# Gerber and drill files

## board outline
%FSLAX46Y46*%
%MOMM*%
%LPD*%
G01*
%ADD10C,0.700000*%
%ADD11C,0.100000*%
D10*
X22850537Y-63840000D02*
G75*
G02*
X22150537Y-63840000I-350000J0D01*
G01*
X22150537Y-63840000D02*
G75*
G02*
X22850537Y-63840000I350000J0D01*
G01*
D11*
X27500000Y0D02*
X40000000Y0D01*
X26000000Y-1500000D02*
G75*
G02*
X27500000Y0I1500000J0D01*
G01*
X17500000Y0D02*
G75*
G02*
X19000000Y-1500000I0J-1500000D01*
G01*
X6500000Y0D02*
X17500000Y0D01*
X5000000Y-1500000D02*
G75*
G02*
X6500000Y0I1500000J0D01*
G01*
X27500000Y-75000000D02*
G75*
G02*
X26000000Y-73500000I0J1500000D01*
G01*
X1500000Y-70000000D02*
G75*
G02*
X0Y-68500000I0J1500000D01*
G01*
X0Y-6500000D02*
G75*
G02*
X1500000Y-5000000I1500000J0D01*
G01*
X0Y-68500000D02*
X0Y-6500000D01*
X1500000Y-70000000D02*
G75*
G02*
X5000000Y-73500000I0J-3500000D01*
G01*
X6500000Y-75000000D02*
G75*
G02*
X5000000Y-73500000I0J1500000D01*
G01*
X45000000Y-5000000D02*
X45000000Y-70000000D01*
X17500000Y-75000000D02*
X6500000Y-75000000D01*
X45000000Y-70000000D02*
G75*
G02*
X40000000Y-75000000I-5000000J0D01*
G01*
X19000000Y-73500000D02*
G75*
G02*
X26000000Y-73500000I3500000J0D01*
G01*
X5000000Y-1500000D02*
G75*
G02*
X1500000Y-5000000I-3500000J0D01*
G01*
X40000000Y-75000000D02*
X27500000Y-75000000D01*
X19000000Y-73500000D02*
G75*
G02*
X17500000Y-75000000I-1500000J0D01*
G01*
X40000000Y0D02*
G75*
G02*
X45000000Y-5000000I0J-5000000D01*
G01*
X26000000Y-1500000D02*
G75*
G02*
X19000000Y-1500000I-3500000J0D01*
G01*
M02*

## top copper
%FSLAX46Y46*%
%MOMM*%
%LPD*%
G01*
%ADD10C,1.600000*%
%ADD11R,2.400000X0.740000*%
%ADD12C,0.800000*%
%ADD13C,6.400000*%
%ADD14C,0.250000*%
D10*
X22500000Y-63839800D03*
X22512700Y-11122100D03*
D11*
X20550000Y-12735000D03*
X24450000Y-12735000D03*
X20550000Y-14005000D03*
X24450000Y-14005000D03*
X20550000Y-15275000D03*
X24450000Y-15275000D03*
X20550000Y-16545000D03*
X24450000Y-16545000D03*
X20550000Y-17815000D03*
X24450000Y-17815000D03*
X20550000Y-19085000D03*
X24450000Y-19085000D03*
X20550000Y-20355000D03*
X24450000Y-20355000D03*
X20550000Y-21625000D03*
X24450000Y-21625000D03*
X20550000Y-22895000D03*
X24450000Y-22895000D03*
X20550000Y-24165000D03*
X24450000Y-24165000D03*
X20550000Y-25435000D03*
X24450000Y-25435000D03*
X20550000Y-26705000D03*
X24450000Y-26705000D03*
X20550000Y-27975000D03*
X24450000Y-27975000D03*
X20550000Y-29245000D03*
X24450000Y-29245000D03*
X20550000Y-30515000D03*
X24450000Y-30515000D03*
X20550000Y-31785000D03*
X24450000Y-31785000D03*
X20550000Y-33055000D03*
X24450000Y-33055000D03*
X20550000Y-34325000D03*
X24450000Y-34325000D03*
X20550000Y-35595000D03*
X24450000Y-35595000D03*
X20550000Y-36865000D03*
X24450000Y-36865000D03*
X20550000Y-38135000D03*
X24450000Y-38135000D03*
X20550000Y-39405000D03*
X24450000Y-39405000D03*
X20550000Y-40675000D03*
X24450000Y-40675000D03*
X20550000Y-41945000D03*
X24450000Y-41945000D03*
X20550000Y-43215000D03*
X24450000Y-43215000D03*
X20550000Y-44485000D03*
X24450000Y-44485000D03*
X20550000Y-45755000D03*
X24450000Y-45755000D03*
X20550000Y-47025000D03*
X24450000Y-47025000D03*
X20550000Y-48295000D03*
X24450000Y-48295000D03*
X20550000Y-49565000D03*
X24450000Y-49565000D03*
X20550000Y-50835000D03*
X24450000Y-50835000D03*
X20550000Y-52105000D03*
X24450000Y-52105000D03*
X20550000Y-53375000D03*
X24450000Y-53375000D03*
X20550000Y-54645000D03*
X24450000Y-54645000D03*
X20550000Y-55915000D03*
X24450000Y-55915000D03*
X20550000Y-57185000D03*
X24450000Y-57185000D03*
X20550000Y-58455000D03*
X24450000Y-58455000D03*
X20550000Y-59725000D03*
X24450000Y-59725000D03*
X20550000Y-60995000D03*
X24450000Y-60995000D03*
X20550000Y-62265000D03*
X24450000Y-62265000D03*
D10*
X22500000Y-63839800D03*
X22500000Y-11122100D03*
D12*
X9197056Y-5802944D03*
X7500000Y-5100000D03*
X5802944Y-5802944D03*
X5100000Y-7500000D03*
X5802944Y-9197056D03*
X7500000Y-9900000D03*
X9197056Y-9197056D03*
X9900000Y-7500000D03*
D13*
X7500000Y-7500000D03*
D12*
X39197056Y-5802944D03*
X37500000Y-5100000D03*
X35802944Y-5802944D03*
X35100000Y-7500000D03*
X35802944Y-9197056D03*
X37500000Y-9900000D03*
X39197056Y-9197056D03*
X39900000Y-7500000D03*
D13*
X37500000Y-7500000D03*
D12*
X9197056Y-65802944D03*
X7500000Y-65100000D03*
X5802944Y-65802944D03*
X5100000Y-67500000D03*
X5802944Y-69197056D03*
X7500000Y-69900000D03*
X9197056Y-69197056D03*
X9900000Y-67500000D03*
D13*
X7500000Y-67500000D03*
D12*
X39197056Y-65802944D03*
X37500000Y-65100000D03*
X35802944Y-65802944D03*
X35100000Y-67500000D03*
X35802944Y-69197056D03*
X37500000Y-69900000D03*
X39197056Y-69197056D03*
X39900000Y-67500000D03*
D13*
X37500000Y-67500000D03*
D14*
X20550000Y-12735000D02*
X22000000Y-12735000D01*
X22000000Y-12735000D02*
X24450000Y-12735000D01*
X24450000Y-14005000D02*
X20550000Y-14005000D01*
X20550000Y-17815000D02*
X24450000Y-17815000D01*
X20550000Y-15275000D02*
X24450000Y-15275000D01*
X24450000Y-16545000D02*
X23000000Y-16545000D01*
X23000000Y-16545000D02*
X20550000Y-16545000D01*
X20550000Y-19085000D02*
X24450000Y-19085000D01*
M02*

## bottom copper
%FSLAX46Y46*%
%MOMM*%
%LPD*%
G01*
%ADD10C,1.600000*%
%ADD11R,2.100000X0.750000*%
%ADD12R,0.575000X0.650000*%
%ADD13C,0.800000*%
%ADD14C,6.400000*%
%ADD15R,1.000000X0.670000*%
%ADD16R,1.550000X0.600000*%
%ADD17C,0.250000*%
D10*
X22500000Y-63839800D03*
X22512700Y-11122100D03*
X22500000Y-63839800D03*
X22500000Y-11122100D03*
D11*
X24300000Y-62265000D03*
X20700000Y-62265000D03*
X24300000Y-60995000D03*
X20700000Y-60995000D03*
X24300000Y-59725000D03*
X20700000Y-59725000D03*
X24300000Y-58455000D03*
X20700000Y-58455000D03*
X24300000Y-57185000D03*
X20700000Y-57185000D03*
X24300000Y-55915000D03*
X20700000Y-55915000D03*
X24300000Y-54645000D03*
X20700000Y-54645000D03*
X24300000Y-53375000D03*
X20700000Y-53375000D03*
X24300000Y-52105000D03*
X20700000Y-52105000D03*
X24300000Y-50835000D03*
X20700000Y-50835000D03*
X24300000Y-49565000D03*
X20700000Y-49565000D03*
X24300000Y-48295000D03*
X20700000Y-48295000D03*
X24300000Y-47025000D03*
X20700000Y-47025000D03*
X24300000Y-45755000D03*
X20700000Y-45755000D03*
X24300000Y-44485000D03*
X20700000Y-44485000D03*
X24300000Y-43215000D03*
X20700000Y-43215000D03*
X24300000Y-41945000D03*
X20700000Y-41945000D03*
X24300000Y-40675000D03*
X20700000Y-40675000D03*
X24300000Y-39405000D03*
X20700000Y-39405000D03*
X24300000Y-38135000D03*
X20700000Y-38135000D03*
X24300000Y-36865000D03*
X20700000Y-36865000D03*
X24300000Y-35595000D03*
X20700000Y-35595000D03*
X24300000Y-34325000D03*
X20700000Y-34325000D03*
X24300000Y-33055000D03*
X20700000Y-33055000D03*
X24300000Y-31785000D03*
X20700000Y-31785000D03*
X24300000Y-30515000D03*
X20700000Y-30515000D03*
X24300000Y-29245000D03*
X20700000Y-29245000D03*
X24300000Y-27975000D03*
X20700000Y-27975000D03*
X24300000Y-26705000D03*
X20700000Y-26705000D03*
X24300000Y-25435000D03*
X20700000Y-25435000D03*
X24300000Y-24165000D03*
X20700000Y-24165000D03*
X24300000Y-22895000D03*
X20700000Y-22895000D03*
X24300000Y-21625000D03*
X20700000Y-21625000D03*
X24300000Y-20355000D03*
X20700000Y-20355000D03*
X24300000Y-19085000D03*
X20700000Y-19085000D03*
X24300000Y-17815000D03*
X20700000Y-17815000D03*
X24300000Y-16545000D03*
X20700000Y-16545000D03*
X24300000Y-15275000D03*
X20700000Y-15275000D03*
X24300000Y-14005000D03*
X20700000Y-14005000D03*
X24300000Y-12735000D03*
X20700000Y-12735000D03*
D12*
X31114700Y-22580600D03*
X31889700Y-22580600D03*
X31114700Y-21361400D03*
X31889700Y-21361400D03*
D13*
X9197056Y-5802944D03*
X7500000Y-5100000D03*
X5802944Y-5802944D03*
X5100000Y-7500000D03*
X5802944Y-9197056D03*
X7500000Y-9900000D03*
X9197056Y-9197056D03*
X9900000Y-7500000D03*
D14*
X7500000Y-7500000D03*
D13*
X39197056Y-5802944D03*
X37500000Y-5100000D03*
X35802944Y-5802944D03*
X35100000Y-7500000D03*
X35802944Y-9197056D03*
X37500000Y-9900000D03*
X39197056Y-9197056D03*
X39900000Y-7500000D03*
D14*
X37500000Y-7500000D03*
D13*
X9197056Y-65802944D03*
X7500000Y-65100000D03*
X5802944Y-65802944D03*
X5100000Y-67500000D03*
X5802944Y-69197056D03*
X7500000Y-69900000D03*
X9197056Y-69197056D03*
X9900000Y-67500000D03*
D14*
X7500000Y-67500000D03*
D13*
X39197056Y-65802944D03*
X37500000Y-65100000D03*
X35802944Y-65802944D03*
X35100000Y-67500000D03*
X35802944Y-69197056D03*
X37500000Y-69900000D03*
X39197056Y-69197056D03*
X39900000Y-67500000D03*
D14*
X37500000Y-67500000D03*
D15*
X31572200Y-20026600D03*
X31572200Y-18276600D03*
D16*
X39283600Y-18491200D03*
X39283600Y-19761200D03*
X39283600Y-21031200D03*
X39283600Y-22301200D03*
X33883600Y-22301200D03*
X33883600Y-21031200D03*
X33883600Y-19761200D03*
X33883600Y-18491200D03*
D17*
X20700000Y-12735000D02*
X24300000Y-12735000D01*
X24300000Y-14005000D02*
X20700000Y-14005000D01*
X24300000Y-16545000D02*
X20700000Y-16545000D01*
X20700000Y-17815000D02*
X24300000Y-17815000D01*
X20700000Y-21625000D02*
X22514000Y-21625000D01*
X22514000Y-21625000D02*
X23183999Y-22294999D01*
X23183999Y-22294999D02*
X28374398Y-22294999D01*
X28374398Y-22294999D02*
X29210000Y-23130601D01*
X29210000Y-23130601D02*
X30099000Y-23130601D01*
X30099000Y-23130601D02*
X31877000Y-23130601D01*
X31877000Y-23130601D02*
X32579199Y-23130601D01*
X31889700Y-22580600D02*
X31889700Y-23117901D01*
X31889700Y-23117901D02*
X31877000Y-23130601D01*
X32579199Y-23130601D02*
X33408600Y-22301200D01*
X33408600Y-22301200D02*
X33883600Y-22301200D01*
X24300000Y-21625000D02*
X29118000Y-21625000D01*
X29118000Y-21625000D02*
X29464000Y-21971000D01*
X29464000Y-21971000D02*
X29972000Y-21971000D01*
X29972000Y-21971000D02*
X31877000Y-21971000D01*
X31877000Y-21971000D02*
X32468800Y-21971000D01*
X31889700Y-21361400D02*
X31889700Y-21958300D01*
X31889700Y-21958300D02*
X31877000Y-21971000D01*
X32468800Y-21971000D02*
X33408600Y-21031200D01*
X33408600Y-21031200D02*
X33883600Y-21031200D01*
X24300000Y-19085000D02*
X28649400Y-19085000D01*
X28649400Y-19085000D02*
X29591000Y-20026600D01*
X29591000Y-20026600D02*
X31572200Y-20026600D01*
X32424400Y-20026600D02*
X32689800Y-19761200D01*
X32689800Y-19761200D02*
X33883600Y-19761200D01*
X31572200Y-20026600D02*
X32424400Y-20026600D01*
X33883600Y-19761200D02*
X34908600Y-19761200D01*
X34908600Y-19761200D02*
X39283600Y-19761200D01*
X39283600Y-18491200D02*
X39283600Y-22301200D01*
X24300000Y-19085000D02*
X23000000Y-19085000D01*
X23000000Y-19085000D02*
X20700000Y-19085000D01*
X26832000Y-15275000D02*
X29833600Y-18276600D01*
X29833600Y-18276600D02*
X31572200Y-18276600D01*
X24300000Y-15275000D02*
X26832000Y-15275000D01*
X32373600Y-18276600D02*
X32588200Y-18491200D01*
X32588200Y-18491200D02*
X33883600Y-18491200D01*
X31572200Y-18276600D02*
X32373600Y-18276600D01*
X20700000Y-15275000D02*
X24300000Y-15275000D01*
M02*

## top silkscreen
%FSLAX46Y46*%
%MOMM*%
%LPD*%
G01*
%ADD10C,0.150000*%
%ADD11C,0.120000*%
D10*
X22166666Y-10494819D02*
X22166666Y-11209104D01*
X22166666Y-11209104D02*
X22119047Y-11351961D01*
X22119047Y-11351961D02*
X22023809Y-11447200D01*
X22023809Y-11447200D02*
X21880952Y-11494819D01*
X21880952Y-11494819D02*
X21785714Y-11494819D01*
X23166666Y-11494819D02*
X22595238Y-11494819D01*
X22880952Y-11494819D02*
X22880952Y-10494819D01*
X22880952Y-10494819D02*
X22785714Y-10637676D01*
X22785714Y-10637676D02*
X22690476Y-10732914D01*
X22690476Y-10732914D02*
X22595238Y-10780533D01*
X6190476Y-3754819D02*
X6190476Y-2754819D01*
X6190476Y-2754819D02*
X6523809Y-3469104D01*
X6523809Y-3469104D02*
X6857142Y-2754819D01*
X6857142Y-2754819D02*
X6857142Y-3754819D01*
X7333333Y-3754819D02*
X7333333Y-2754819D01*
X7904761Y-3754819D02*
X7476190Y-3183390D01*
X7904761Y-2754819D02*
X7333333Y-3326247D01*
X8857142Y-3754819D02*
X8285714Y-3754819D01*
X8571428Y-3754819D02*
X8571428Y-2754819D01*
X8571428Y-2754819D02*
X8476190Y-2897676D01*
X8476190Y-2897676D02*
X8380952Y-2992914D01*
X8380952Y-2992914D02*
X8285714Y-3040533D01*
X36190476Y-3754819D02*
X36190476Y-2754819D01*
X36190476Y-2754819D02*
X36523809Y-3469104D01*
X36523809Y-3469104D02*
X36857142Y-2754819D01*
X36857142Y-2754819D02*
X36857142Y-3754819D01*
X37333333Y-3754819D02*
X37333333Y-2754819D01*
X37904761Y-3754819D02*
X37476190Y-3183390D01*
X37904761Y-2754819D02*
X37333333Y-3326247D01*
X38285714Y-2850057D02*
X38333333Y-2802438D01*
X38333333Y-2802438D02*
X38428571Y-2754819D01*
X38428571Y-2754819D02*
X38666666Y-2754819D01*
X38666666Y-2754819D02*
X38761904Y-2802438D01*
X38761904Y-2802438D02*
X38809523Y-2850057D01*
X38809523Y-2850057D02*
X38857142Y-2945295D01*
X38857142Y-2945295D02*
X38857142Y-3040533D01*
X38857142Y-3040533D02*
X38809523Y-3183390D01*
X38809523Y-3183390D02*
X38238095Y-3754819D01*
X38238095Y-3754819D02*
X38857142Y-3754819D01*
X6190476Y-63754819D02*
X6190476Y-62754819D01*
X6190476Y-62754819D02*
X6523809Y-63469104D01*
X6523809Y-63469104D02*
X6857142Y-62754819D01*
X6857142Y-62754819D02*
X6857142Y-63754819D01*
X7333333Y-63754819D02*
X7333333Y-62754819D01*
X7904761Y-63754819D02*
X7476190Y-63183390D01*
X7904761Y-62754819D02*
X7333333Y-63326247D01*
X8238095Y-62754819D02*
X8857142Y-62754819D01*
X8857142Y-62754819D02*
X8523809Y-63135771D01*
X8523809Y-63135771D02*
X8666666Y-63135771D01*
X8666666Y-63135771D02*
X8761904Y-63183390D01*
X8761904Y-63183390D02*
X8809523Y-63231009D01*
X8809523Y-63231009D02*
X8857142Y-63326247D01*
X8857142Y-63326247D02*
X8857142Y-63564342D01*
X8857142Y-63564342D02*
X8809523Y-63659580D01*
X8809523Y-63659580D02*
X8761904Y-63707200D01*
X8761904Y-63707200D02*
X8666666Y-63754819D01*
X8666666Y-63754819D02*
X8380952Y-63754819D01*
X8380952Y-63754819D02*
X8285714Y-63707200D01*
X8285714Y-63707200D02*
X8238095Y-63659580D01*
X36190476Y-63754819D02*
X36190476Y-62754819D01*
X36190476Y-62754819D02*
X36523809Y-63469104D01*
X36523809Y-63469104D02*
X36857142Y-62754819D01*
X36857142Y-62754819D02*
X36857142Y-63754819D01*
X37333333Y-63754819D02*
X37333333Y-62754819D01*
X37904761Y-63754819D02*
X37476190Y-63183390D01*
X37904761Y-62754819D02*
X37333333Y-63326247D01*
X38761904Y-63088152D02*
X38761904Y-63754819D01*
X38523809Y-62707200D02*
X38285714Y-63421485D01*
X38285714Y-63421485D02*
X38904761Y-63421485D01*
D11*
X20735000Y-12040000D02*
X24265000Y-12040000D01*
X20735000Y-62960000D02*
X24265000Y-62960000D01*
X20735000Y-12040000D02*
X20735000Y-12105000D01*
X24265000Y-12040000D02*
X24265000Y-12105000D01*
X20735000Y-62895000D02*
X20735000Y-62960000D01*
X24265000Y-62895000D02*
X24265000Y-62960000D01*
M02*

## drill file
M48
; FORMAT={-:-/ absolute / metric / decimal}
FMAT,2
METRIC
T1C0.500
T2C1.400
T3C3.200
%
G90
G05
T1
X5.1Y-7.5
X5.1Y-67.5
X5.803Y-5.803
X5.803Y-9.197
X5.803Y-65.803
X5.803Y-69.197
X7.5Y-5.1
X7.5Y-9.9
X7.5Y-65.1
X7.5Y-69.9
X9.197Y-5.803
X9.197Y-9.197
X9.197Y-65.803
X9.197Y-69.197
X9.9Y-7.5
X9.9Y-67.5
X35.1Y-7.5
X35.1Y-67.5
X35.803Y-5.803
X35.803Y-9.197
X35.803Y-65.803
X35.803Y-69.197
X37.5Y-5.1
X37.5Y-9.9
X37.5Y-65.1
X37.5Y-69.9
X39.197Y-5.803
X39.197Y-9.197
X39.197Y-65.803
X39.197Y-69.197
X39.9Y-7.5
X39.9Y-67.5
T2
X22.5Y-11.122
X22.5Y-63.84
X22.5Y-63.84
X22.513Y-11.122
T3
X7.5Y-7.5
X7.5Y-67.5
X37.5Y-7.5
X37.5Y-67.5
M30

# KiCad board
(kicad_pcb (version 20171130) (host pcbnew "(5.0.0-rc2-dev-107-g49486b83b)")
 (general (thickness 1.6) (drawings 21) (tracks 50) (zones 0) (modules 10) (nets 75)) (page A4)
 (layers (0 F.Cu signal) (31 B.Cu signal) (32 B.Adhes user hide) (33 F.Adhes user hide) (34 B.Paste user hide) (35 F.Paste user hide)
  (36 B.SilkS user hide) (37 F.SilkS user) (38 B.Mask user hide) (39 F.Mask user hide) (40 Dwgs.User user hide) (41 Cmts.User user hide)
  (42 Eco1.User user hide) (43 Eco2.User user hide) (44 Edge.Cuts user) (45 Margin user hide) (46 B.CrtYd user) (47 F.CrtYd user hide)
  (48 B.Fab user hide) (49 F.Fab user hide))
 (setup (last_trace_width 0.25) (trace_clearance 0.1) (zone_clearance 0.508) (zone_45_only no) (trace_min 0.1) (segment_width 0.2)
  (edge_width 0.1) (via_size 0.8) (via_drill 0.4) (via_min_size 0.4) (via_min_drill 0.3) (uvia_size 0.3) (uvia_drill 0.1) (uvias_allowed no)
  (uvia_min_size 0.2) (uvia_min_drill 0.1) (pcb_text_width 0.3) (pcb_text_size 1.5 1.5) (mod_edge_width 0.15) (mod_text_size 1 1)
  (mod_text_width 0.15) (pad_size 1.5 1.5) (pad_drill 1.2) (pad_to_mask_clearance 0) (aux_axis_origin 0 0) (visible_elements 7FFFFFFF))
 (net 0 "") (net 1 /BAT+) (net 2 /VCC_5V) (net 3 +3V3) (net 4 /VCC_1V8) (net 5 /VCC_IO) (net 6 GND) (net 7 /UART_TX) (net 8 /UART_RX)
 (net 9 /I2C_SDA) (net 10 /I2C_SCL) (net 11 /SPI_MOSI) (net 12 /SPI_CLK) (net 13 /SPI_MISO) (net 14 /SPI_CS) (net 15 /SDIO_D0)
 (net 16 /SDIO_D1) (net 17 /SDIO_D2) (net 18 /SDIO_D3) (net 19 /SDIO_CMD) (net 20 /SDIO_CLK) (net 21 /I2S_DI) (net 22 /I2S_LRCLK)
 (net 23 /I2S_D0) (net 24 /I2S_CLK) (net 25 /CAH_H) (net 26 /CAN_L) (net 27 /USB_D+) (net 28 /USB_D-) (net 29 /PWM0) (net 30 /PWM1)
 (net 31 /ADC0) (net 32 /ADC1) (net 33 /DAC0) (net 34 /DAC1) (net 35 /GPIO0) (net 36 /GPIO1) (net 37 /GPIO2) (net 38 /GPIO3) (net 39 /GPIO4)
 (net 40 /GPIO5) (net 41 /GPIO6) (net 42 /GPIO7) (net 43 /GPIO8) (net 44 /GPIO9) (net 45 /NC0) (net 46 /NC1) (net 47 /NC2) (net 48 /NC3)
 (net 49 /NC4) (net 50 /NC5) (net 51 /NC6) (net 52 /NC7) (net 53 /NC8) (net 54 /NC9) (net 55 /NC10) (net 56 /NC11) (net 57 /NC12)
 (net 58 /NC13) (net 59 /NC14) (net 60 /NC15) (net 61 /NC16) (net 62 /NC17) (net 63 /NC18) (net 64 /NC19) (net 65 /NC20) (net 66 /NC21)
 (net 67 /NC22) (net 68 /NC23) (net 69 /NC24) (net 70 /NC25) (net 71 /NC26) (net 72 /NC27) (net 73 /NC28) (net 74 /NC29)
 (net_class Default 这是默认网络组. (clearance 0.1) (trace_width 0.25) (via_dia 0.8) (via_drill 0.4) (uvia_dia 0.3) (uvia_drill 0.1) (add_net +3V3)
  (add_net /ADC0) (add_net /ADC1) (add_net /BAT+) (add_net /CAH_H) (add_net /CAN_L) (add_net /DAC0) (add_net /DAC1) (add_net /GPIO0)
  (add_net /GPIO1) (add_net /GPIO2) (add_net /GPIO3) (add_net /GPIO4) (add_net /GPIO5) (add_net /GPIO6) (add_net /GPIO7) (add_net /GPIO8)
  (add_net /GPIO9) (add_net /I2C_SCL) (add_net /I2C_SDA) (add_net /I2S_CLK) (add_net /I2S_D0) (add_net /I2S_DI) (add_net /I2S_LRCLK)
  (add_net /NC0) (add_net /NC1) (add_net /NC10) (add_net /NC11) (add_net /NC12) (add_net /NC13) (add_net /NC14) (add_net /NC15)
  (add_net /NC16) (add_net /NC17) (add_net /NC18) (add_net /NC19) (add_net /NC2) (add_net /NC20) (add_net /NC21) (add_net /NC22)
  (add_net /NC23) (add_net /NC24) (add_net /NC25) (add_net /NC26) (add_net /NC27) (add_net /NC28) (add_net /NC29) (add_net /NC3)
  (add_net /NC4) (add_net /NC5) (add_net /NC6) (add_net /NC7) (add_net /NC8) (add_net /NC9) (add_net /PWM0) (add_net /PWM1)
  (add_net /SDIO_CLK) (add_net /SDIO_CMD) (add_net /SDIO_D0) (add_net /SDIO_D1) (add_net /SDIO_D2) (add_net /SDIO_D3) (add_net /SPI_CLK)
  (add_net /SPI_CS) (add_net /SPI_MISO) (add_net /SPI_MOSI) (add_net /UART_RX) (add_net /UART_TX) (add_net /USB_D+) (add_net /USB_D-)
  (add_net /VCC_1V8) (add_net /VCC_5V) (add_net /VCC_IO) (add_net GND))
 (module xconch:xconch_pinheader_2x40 (layer F.Cu) (at 22.5 37.5)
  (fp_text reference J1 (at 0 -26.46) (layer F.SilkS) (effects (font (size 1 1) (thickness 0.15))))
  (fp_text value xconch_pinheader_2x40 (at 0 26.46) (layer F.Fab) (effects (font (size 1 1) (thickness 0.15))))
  (fp_line (start -1.765 -25.46) (end 1.765 -25.46) (layer F.SilkS) (width 0.12))
  (fp_line (start -1.765 25.46) (end 1.765 25.46) (layer F.SilkS) (width 0.12))
  (fp_line (start -1.765 -25.46) (end -1.765 -25.395) (layer F.SilkS) (width 0.12))
  (fp_line (start 1.765 -25.46) (end 1.765 -25.395) (layer F.SilkS) (width 0.12))
  (fp_line (start -1.765 25.395) (end -1.765 25.46) (layer F.SilkS) (width 0.12))
  (fp_line (start 1.765 25.395) (end 1.765 25.46) (layer F.SilkS) (width 0.12))
  (pad "" thru_hole circle (at 0 26.3398) (size 1.6 1.6) (drill 1.4) (layers *.Cu *.Mask))
  (pad "" thru_hole circle (at 0.0127 -26.3779) (size 1.6 1.6) (drill 1.4) (layers *.Cu *.Mask))
  (pad 1 smd rect (at -1.95 -24.765) (size 2.4 0.74) (layers F.Cu F.Paste F.Mask) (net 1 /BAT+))
  (pad 2 smd rect (at 1.95 -24.765) (size 2.4 0.74) (layers F.Cu F.Paste F.Mask) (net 1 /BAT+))
  (pad 3 smd rect (at -1.95 -23.495) (size 2.4 0.74) (layers F.Cu F.Paste F.Mask) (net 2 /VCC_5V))
  (pad 4 smd rect (at 1.95 -23.495) (size 2.4 0.74) (layers F.Cu F.Paste F.Mask) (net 2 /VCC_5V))
  (pad 5 smd rect (at -1.95 -22.225) (size 2.4 0.74) (layers F.Cu F.Paste F.Mask) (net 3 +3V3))
  (pad 6 smd rect (at 1.95 -22.225) (size 2.4 0.74) (layers F.Cu F.Paste F.Mask) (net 3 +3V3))
  (pad 7 smd rect (at -1.95 -20.955) (size 2.4 0.74) (layers F.Cu F.Paste F.Mask) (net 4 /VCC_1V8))
  (pad 8 smd rect (at 1.95 -20.955) (size 2.4 0.74) (layers F.Cu F.Paste F.Mask) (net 4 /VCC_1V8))
  (pad 9 smd rect (at -1.95 -19.685) (size 2.4 0.74) (layers F.Cu F.Paste F.Mask) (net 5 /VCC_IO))
  (pad 10 smd rect (at 1.95 -19.685) (size 2.4 0.74) (layers F.Cu F.Paste F.Mask) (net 5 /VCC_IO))
  (pad 11 smd rect (at -1.95 -18.415) (size 2.4 0.74) (layers F.Cu F.Paste F.Mask) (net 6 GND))
  (pad 12 smd rect (at 1.95 -18.415) (size 2.4 0.74) (layers F.Cu F.Paste F.Mask) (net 6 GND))
  (pad 13 smd rect (at -1.95 -17.145) (size 2.4 0.74) (layers F.Cu F.Paste F.Mask) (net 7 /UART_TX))
  (pad 14 smd rect (at 1.95 -17.145) (size 2.4 0.74) (layers F.Cu F.Paste F.Mask) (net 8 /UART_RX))
  (pad 15 smd rect (at -1.95 -15.875) (size 2.4 0.74) (layers F.Cu F.Paste F.Mask) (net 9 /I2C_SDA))
  (pad 16 smd rect (at 1.95 -15.875) (size 2.4 0.74) (layers F.Cu F.Paste F.Mask) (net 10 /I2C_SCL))
  (pad 17 smd rect (at -1.95 -14.605) (size 2.4 0.74) (layers F.Cu F.Paste F.Mask) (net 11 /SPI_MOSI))
  (pad 18 smd rect (at 1.95 -14.605) (size 2.4 0.74) (layers F.Cu F.Paste F.Mask) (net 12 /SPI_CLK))
  (pad 19 smd rect (at -1.95 -13.335) (size 2.4 0.74) (layers F.Cu F.Paste F.Mask) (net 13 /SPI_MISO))
  (pad 20 smd rect (at 1.95 -13.335) (size 2.4 0.74) (layers F.Cu F.Paste F.Mask) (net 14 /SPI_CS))
  (pad 21 smd rect (at -1.95 -12.065) (size 2.4 0.74) (layers F.Cu F.Paste F.Mask) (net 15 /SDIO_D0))
  (pad 22 smd rect (at 1.95 -12.065) (size 2.4 0.74) (layers F.Cu F.Paste F.Mask) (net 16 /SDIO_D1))
  (pad 23 smd rect (at -1.95 -10.795) (size 2.4 0.74) (layers F.Cu F.Paste F.Mask) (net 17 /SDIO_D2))
  (pad 24 smd rect (at 1.95 -10.795) (size 2.4 0.74) (layers F.Cu F.Paste F.Mask) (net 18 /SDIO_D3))
  (pad 25 smd rect (at -1.95 -9.525) (size 2.4 0.74) (layers F.Cu F.Paste F.Mask) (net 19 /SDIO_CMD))
  (pad 26 smd rect (at 1.95 -9.525) (size 2.4 0.74) (layers F.Cu F.Paste F.Mask) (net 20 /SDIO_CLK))
  (pad 27 smd rect (at -1.95 -8.255) (size 2.4 0.74) (layers F.Cu F.Paste F.Mask) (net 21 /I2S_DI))
  (pad 28 smd rect (at 1.95 -8.255) (size 2.4 0.74) (layers F.Cu F.Paste F.Mask) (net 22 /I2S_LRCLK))
  (pad 29 smd rect (at -1.95 -6.985) (size 2.4 0.74) (layers F.Cu F.Paste F.Mask) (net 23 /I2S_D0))
  (pad 30 smd rect (at 1.95 -6.985) (size 2.4 0.74) (layers F.Cu F.Paste F.Mask) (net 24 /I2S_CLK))
  (pad 31 smd rect (at -1.95 -5.715) (size 2.4 0.74) (layers F.Cu F.Paste F.Mask) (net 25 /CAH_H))
  (pad 32 smd rect (at 1.95 -5.715) (size 2.4 0.74) (layers F.Cu F.Paste F.Mask) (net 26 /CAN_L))
  (pad 33 smd rect (at -1.95 -4.445) (size 2.4 0.74) (layers F.Cu F.Paste F.Mask) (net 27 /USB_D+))
  (pad 34 smd rect (at 1.95 -4.445) (size 2.4 0.74) (layers F.Cu F.Paste F.Mask) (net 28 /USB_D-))
  (pad 35 smd rect (at -1.95 -3.175) (size 2.4 0.74) (layers F.Cu F.Paste F.Mask) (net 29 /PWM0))
  (pad 36 smd rect (at 1.95 -3.175) (size 2.4 0.74) (layers F.Cu F.Paste F.Mask) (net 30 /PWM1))
  (pad 37 smd rect (at -1.95 -1.905) (size 2.4 0.74) (layers F.Cu F.Paste F.Mask) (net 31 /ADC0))
  (pad 38 smd rect (at 1.95 -1.905) (size 2.4 0.74) (layers F.Cu F.Paste F.Mask) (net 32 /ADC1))
  (pad 39 smd rect (at -1.95 -0.635) (size 2.4 0.74) (layers F.Cu F.Paste F.Mask) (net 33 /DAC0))
  (pad 40 smd rect (at 1.95 -0.635) (size 2.4 0.74) (layers F.Cu F.Paste F.Mask) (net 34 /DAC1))
  (pad 41 smd rect (at -1.95 0.635) (size 2.4 0.74) (layers F.Cu F.Paste F.Mask) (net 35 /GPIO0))
  (pad 42 smd rect (at 1.95 0.635) (size 2.4 0.74) (layers F.Cu F.Paste F.Mask) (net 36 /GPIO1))
  (pad 43 smd rect (at -1.95 1.905) (size 2.4 0.74) (layers F.Cu F.Paste F.Mask) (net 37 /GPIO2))
  (pad 44 smd rect (at 1.95 1.905) (size 2.4 0.74) (layers F.Cu F.Paste F.Mask) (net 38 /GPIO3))
  (pad 45 smd rect (at -1.95 3.175) (size 2.4 0.74) (layers F.Cu F.Paste F.Mask) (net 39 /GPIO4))
  (pad 46 smd rect (at 1.95 3.175) (size 2.4 0.74) (layers F.Cu F.Paste F.Mask) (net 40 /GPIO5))
  (pad 47 smd rect (at -1.95 4.445) (size 2.4 0.74) (layers F.Cu F.Paste F.Mask) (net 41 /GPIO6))
  (pad 48 smd rect (at 1.95 4.445) (size 2.4 0.74) (layers F.Cu F.Paste F.Mask) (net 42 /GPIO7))
  (pad 49 smd rect (at -1.95 5.715) (size 2.4 0.74) (layers F.Cu F.Paste F.Mask) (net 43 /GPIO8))
  (pad 50 smd rect (at 1.95 5.715) (size 2.4 0.74) (layers F.Cu F.Paste F.Mask) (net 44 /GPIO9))
  (pad 51 smd rect (at -1.95 6.985) (size 2.4 0.74) (layers F.Cu F.Paste F.Mask) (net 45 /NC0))
  (pad 52 smd rect (at 1.95 6.985) (size 2.4 0.74) (layers F.Cu F.Paste F.Mask) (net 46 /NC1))
  (pad 53 smd rect (at -1.95 8.255) (size 2.4 0.74) (layers F.Cu F.Paste F.Mask) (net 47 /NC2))
  (pad 54 smd rect (at 1.95 8.255) (size 2.4 0.74) (layers F.Cu F.Paste F.Mask) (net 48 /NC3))
  (pad 55 smd rect (at -1.95 9.525) (size 2.4 0.74) (layers F.Cu F.Paste F.Mask) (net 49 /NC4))
  (pad 56 smd rect (at 1.95 9.525) (size 2.4 0.74) (layers F.Cu F.Paste F.Mask) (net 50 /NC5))
  (pad 57 smd rect (at -1.95 10.795) (size 2.4 0.74) (layers F.Cu F.Paste F.Mask) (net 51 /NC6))
  (pad 58 smd rect (at 1.95 10.795) (size 2.4 0.74) (layers F.Cu F.Paste F.Mask) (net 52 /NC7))
  (pad 59 smd rect (at -1.95 12.065) (size 2.4 0.74) (layers F.Cu F.Paste F.Mask) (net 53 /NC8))
  (pad 60 smd rect (at 1.95 12.065) (size 2.4 0.74) (layers F.Cu F.Paste F.Mask) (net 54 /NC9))
  (pad 61 smd rect (at -1.95 13.335) (size 2.4 0.74) (layers F.Cu F.Paste F.Mask) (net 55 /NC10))
  (pad 62 smd rect (at 1.95 13.335) (size 2.4 0.74) (layers F.Cu F.Paste F.Mask) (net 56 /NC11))
  (pad 63 smd rect (at -1.95 14.605) (size 2.4 0.74) (layers F.Cu F.Paste F.Mask) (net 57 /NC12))
  (pad 64 smd rect (at 1.95 14.605) (size 2.4 0.74) (layers F.Cu F.Paste F.Mask) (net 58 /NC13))
  (pad 65 smd rect (at -1.95 15.875) (size 2.4 0.74) (layers F.Cu F.Paste F.Mask) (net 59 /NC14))
  (pad 66 smd rect (at 1.95 15.875) (size 2.4 0.74) (layers F.Cu F.Paste F.Mask) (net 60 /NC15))
  (pad 67 smd rect (at -1.95 17.145) (size 2.4 0.74) (layers F.Cu F.Paste F.Mask) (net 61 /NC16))
  (pad 68 smd rect (at 1.95 17.145) (size 2.4 0.74) (layers F.Cu F.Paste F.Mask) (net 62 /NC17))
  (pad 69 smd rect (at -1.95 18.415) (size 2.4 0.74) (layers F.Cu F.Paste F.Mask) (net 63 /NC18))
  (pad 70 smd rect (at 1.95 18.415) (size 2.4 0.74) (layers F.Cu F.Paste F.Mask) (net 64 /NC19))
  (pad 71 smd rect (at -1.95 19.685) (size 2.4 0.74) (layers F.Cu F.Paste F.Mask) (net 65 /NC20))
  (pad 72 smd rect (at 1.95 19.685) (size 2.4 0.74) (layers F.Cu F.Paste F.Mask) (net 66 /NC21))
  (pad 73 smd rect (at -1.95 20.955) (size 2.4 0.74) (layers F.Cu F.Paste F.Mask) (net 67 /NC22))
  (pad 74 smd rect (at 1.95 20.955) (size 2.4 0.74) (layers F.Cu F.Paste F.Mask) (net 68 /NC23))
  (pad 75 smd rect (at -1.95 22.225) (size 2.4 0.74) (layers F.Cu F.Paste F.Mask) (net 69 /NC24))
  (pad 76 smd rect (at 1.95 22.225) (size 2.4 0.74) (layers F.Cu F.Paste F.Mask) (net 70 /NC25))
  (pad 77 smd rect (at -1.95 23.495) (size 2.4 0.74) (layers F.Cu F.Paste F.Mask) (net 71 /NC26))
  (pad 78 smd rect (at 1.95 23.495) (size 2.4 0.74) (layers F.Cu F.Paste F.Mask) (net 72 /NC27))
  (pad 79 smd rect (at -1.95 24.765) (size 2.4 0.74) (layers F.Cu F.Paste F.Mask) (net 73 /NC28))
  (pad 80 smd rect (at 1.95 24.765) (size 2.4 0.74) (layers F.Cu F.Paste F.Mask) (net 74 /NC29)))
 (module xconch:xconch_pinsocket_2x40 (layer B.Cu) (at 22.5 37.5 180)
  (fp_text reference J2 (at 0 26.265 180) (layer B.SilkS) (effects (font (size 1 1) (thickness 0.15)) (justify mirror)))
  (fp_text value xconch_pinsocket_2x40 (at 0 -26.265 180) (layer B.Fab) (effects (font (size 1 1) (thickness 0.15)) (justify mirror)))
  (pad "" thru_hole circle (at 0 -26.3398 180) (size 1.6 1.6) (drill 1.4) (layers *.Cu *.Mask))
  (pad "" thru_hole circle (at 0 26.3779 180) (size 1.6 1.6) (drill 1.4) (layers *.Cu *.Mask))
  (pad 79 smd rect (at -1.8 -24.765 180) (size 2.1 0.75) (layers B.Cu B.Paste B.Mask) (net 74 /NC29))
  (pad 80 smd rect (at 1.8 -24.765 180) (size 2.1 0.75) (layers B.Cu B.Paste B.Mask) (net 73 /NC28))
  (pad 77 smd rect (at -1.8 -23.495 180) (size 2.1 0.75) (layers B.Cu B.Paste B.Mask) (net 72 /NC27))
  (pad 78 smd rect (at 1.8 -23.495 180) (size 2.1 0.75) (layers B.Cu B.Paste B.Mask) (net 71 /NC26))
  (pad 75 smd rect (at -1.8 -22.225 180) (size 2.1 0.75) (layers B.Cu B.Paste B.Mask) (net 70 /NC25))
  (pad 76 smd rect (at 1.8 -22.225 180) (size 2.1 0.75) (layers B.Cu B.Paste B.Mask) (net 69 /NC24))
  (pad 73 smd rect (at -1.8 -20.955 180) (size 2.1 0.75) (layers B.Cu B.Paste B.Mask) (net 68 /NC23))
  (pad 74 smd rect (at 1.8 -20.955 180) (size 2.1 0.75) (layers B.Cu B.Paste B.Mask) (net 67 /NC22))
  (pad 71 smd rect (at -1.8 -19.685 180) (size 2.1 0.75) (layers B.Cu B.Paste B.Mask) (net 66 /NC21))
  (pad 72 smd rect (at 1.8 -19.685 180) (size 2.1 0.75) (layers B.Cu B.Paste B.Mask) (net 65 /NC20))
  (pad 69 smd rect (at -1.8 -18.415 180) (size 2.1 0.75) (layers B.Cu B.Paste B.Mask) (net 64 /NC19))
  (pad 70 smd rect (at 1.8 -18.415 180) (size 2.1 0.75) (layers B.Cu B.Paste B.Mask) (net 63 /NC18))
  (pad 67 smd rect (at -1.8 -17.145 180) (size 2.1 0.75) (layers B.Cu B.Paste B.Mask) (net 62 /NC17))
  (pad 68 smd rect (at 1.8 -17.145 180) (size 2.1 0.75) (layers B.Cu B.Paste B.Mask) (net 61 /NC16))
  (pad 65 smd rect (at -1.8 -15.875 180) (size 2.1 0.75) (layers B.Cu B.Paste B.Mask) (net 60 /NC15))
  (pad 66 smd rect (at 1.8 -15.875 180) (size 2.1 0.75) (layers B.Cu B.Paste B.Mask) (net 59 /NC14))
  (pad 63 smd rect (at -1.8 -14.605 180) (size 2.1 0.75) (layers B.Cu B.Paste B.Mask) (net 58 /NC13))
  (pad 64 smd rect (at 1.8 -14.605 180) (size 2.1 0.75) (layers B.Cu B.Paste B.Mask) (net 57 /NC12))
  (pad 61 smd rect (at -1.8 -13.335 180) (size 2.1 0.75) (layers B.Cu B.Paste B.Mask) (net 56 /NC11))
  (pad 62 smd rect (at 1.8 -13.335 180) (size 2.1 0.75) (layers B.Cu B.Paste B.Mask) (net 55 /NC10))
  (pad 59 smd rect (at -1.8 -12.065 180) (size 2.1 0.75) (layers B.Cu B.Paste B.Mask) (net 54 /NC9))
  (pad 60 smd rect (at 1.8 -12.065 180) (size 2.1 0.75) (layers B.Cu B.Paste B.Mask) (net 53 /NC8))
  (pad 57 smd rect (at -1.8 -10.795 180) (size 2.1 0.75) (layers B.Cu B.Paste B.Mask) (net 52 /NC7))
  (pad 58 smd rect (at 1.8 -10.795 180) (size 2.1 0.75) (layers B.Cu B.Paste B.Mask) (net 51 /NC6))
  (pad 55 smd rect (at -1.8 -9.525 180) (size 2.1 0.75) (layers B.Cu B.Paste B.Mask) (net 50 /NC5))
  (pad 56 smd rect (at 1.8 -9.525 180) (size 2.1 0.75) (layers B.Cu B.Paste B.Mask) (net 49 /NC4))
  (pad 53 smd rect (at -1.8 -8.255 180) (size 2.1 0.75) (layers B.Cu B.Paste B.Mask) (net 48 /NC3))
  (pad 54 smd rect (at 1.8 -8.255 180) (size 2.1 0.75) (layers B.Cu B.Paste B.Mask) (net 47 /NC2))
  (pad 51 smd rect (at -1.8 -6.985 180) (size 2.1 0.75) (layers B.Cu B.Paste B.Mask) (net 46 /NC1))
  (pad 52 smd rect (at 1.8 -6.985 180) (size 2.1 0.75) (layers B.Cu B.Paste B.Mask) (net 45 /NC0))
  (pad 49 smd rect (at -1.8 -5.715 180) (size 2.1 0.75) (layers B.Cu B.Paste B.Mask) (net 44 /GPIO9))
  (pad 50 smd rect (at 1.8 -5.715 180) (size 2.1 0.75) (layers B.Cu B.Paste B.Mask) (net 43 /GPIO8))
  (pad 47 smd rect (at -1.8 -4.445 180) (size 2.1 0.75) (layers B.Cu B.Paste B.Mask) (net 42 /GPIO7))
  (pad 48 smd rect (at 1.8 -4.445 180) (size 2.1 0.75) (layers B.Cu B.Paste B.Mask) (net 41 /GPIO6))
  (pad 45 smd rect (at -1.8 -3.175 180) (size 2.1 0.75) (layers B.Cu B.Paste B.Mask) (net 40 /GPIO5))
  (pad 46 smd rect (at 1.8 -3.175 180) (size 2.1 0.75) (layers B.Cu B.Paste B.Mask) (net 39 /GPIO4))
  (pad 43 smd rect (at -1.8 -1.905 180) (size 2.1 0.75) (layers B.Cu B.Paste B.Mask) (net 38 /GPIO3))
  (pad 44 smd rect (at 1.8 -1.905 180) (size 2.1 0.75) (layers B.Cu B.Paste B.Mask) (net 37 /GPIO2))
  (pad 41 smd rect (at -1.8 -0.635 180) (size 2.1 0.75) (layers B.Cu B.Paste B.Mask) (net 36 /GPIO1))
  (pad 42 smd rect (at 1.8 -0.635 180) (size 2.1 0.75) (layers B.Cu B.Paste B.Mask) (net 35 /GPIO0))
  (pad 39 smd rect (at -1.8 0.635 180) (size 2.1 0.75) (layers B.Cu B.Paste B.Mask) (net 34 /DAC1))
  (pad 40 smd rect (at 1.8 0.635 180) (size 2.1 0.75) (layers B.Cu B.Paste B.Mask) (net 33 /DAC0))
  (pad 37 smd rect (at -1.8 1.905 180) (size 2.1 0.75) (layers B.Cu B.Paste B.Mask) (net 32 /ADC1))
  (pad 38 smd rect (at 1.8 1.905 180) (size 2.1 0.75) (layers B.Cu B.Paste B.Mask) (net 31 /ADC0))
  (pad 35 smd rect (at -1.8 3.175 180) (size 2.1 0.75) (layers B.Cu B.Paste B.Mask) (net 30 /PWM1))
  (pad 36 smd rect (at 1.8 3.175 180) (size 2.1 0.75) (layers B.Cu B.Paste B.Mask) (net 29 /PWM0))
  (pad 33 smd rect (at -1.8 4.445 180) (size 2.1 0.75) (layers B.Cu B.Paste B.Mask) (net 28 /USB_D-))
  (pad 34 smd rect (at 1.8 4.445 180) (size 2.1 0.75) (layers B.Cu B.Paste B.Mask) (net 27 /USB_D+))
  (pad 31 smd rect (at -1.8 5.715 180) (size 2.1 0.75) (layers B.Cu B.Paste B.Mask) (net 26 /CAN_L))
  (pad 32 smd rect (at 1.8 5.715 180) (size 2.1 0.75) (layers B.Cu B.Paste B.Mask) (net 25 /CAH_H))
  (pad 29 smd rect (at -1.8 6.985 180) (size 2.1 0.75) (layers B.Cu B.Paste B.Mask) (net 24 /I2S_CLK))
  (pad 30 smd rect (at 1.8 6.985 180) (size 2.1 0.75) (layers B.Cu B.Paste B.Mask) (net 23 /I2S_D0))
  (pad 27 smd rect (at -1.8 8.255 180) (size 2.1 0.75) (layers B.Cu B.Paste B.Mask) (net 22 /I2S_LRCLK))
  (pad 28 smd rect (at 1.8 8.255 180) (size 2.1 0.75) (layers B.Cu B.Paste B.Mask) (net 21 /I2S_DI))
  (pad 25 smd rect (at -1.8 9.525 180) (size 2.1 0.75) (layers B.Cu B.Paste B.Mask) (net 20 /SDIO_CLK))
  (pad 26 smd rect (at 1.8 9.525 180) (size 2.1 0.75) (layers B.Cu B.Paste B.Mask) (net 19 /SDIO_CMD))
  (pad 23 smd rect (at -1.8 10.795 180) (size 2.1 0.75) (layers B.Cu B.Paste B.Mask) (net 18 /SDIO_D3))
  (pad 24 smd rect (at 1.8 10.795 180) (size 2.1 0.75) (layers B.Cu B.Paste B.Mask) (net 17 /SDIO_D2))
  (pad 21 smd rect (at -1.8 12.065 180) (size 2.1 0.75) (layers B.Cu B.Paste B.Mask) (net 16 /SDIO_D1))
  (pad 22 smd rect (at 1.8 12.065 180) (size 2.1 0.75) (layers B.Cu B.Paste B.Mask) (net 15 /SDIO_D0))
  (pad 19 smd rect (at -1.8 13.335 180) (size 2.1 0.75) (layers B.Cu B.Paste B.Mask) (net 14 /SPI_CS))
  (pad 20 smd rect (at 1.8 13.335 180) (size 2.1 0.75) (layers B.Cu B.Paste B.Mask) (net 13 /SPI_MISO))
  (pad 17 smd rect (at -1.8 14.605 180) (size 2.1 0.75) (layers B.Cu B.Paste B.Mask) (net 12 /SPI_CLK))
  (pad 18 smd rect (at 1.8 14.605 180) (size 2.1 0.75) (layers B.Cu B.Paste B.Mask) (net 11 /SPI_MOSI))
  (pad 15 smd rect (at -1.8 15.875 180) (size 2.1 0.75) (layers B.Cu B.Paste B.Mask) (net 10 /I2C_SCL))
  (pad 16 smd rect (at 1.8 15.875 180) (size 2.1 0.75) (layers B.Cu B.Paste B.Mask) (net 9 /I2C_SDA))
  (pad 13 smd rect (at -1.8 17.145 180) (size 2.1 0.75) (layers B.Cu B.Paste B.Mask) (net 8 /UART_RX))
  (pad 14 smd rect (at 1.8 17.145 180) (size 2.1 0.75) (layers B.Cu B.Paste B.Mask) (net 7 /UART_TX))
  (pad 11 smd rect (at -1.8 18.415 180) (size 2.1 0.75) (layers B.Cu B.Paste B.Mask) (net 6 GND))
  (pad 12 smd rect (at 1.8 18.415 180) (size 2.1 0.75) (layers B.Cu B.Paste B.Mask) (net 6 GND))
  (pad 9 smd rect (at -1.8 19.685 180) (size 2.1 0.75) (layers B.Cu B.Paste B.Mask) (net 5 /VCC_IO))
  (pad 10 smd rect (at 1.8 19.685 180) (size 2.1 0.75) (layers B.Cu B.Paste B.Mask) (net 5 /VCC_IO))
  (pad 7 smd rect (at -1.8 20.955 180) (size 2.1 0.75) (layers B.Cu B.Paste B.Mask) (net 4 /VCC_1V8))
  (pad 8 smd rect (at 1.8 20.955 180) (size 2.1 0.75) (layers B.Cu B.Paste B.Mask) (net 4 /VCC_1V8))
  (pad 5 smd rect (at -1.8 22.225 180) (size 2.1 0.75) (layers B.Cu B.Paste B.Mask) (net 3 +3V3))
  (pad 6 smd rect (at 1.8 22.225 180) (size 2.1 0.75) (layers B.Cu B.Paste B.Mask) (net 3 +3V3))
  (pad 3 smd rect (at -1.8 23.495 180) (size 2.1 0.75) (layers B.Cu B.Paste B.Mask) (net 2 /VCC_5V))
  (pad 4 smd rect (at 1.8 23.495 180) (size 2.1 0.75) (layers B.Cu B.Paste B.Mask) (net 2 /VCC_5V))
  (pad 1 smd rect (at -1.8 24.765 180) (size 2.1 0.75) (layers B.Cu B.Paste B.Mask) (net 1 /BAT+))
  (pad 2 smd rect (at 1.8 24.765 180) (size 2.1 0.75) (layers B.Cu B.Paste B.Mask) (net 1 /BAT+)))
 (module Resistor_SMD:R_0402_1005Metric (layer B.Cu) (at 31.5022 22.5806)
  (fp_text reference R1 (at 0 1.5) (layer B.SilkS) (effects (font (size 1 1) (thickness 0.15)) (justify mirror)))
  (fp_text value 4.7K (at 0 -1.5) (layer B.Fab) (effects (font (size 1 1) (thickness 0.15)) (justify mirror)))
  (pad 1 smd rect (at -0.3875 0) (size 0.575 0.65) (layers B.Cu B.Paste B.Mask) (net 3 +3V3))
  (pad 2 smd rect (at 0.3875 0) (size 0.575 0.65) (layers B.Cu B.Paste B.Mask) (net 9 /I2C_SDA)))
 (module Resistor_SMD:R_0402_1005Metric (layer B.Cu) (at 31.5022 21.3614)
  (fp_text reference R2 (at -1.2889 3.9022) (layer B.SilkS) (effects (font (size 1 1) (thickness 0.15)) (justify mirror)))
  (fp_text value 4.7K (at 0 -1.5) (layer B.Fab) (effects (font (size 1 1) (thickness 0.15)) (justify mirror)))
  (pad 1 smd rect (at -0.3875 0) (size 0.575 0.65) (layers B.Cu B.Paste B.Mask) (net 3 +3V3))
  (pad 2 smd rect (at 0.3875 0) (size 0.575 0.65) (layers B.Cu B.Paste B.Mask) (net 10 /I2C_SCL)))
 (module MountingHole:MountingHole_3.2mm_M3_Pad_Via (layer F.Cu) (at 7.5 7.5)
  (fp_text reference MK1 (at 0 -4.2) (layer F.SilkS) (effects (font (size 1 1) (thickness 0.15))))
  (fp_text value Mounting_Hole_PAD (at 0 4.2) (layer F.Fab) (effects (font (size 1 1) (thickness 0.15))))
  (pad 1 thru_hole circle (at 1.697056 -1.697056) (size 0.8 0.8) (drill 0.5) (layers *.Cu *.Mask) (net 6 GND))
  (pad 1 thru_hole circle (at 0 -2.4) (size 0.8 0.8) (drill 0.5) (layers *.Cu *.Mask) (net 6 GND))
  (pad 1 thru_hole circle (at -1.697056 -1.697056) (size 0.8 0.8) (drill 0.5) (layers *.Cu *.Mask) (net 6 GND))
  (pad 1 thru_hole circle (at -2.4 0) (size 0.8 0.8) (drill 0.5) (layers *.Cu *.Mask) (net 6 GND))
  (pad 1 thru_hole circle (at -1.697056 1.697056) (size 0.8 0.8) (drill 0.5) (layers *.Cu *.Mask) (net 6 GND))
  (pad 1 thru_hole circle (at 0 2.4) (size 0.8 0.8) (drill 0.5) (layers *.Cu *.Mask) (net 6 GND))
  (pad 1 thru_hole circle (at 1.697056 1.697056) (size 0.8 0.8) (drill 0.5) (layers *.Cu *.Mask) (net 6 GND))
  (pad 1 thru_hole circle (at 2.4 0) (size 0.8 0.8) (drill 0.5) (layers *.Cu *.Mask) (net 6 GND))
  (pad 1 thru_hole circle (at 0 0) (size 6.4 6.4) (drill 3.2) (layers *.Cu *.Mask) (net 6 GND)))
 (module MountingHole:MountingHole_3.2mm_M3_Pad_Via (layer F.Cu) (at 37.5 7.5)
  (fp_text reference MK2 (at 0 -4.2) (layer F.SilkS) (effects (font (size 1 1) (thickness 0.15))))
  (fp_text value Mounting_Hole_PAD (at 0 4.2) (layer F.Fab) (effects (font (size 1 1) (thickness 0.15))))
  (pad 1 thru_hole circle (at 1.697056 -1.697056) (size 0.8 0.8) (drill 0.5) (layers *.Cu *.Mask) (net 6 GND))
  (pad 1 thru_hole circle (at 0 -2.4) (size 0.8 0.8) (drill 0.5) (layers *.Cu *.Mask) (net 6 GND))
  (pad 1 thru_hole circle (at -1.697056 -1.697056) (size 0.8 0.8) (drill 0.5) (layers *.Cu *.Mask) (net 6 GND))
  (pad 1 thru_hole circle (at -2.4 0) (size 0.8 0.8) (drill 0.5) (layers *.Cu *.Mask) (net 6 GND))
  (pad 1 thru_hole circle (at -1.697056 1.697056) (size 0.8 0.8) (drill 0.5) (layers *.Cu *.Mask) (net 6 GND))
  (pad 1 thru_hole circle (at 0 2.4) (size 0.8 0.8) (drill 0.5) (layers *.Cu *.Mask) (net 6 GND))
  (pad 1 thru_hole circle (at 1.697056 1.697056) (size 0.8 0.8) (drill 0.5) (layers *.Cu *.Mask) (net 6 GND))
  (pad 1 thru_hole circle (at 2.4 0) (size 0.8 0.8) (drill 0.5) (layers *.Cu *.Mask) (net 6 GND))
  (pad 1 thru_hole circle (at 0 0) (size 6.4 6.4) (drill 3.2) (layers *.Cu *.Mask) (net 6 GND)))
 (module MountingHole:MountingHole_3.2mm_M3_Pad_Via (layer F.Cu) (at 7.5 67.5)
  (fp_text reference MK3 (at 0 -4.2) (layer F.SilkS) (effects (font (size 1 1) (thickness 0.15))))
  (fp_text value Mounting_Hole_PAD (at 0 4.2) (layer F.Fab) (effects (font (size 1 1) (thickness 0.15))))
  (pad 1 thru_hole circle (at 1.697056 -1.697056) (size 0.8 0.8) (drill 0.5) (layers *.Cu *.Mask) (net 6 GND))
  (pad 1 thru_hole circle (at 0 -2.4) (size 0.8 0.8) (drill 0.5) (layers *.Cu *.Mask) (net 6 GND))
  (pad 1 thru_hole circle (at -1.697056 -1.697056) (size 0.8 0.8) (drill 0.5) (layers *.Cu *.Mask) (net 6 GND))
  (pad 1 thru_hole circle (at -2.4 0) (size 0.8 0.8) (drill 0.5) (layers *.Cu *.Mask) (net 6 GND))
  (pad 1 thru_hole circle (at -1.697056 1.697056) (size 0.8 0.8) (drill 0.5) (layers *.Cu *.Mask) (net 6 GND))
  (pad 1 thru_hole circle (at 0 2.4) (size 0.8 0.8) (drill 0.5) (layers *.Cu *.Mask) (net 6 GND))
  (pad 1 thru_hole circle (at 1.697056 1.697056) (size 0.8 0.8) (drill 0.5) (layers *.Cu *.Mask) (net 6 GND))
  (pad 1 thru_hole circle (at 2.4 0) (size 0.8 0.8) (drill 0.5) (layers *.Cu *.Mask) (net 6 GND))
  (pad 1 thru_hole circle (at 0 0) (size 6.4 6.4) (drill 3.2) (layers *.Cu *.Mask) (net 6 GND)))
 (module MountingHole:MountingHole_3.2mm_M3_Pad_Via (layer F.Cu) (at 37.5 67.5)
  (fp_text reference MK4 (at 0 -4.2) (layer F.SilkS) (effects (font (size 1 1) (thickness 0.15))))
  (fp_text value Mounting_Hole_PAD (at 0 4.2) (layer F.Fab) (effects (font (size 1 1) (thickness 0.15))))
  (pad 1 thru_hole circle (at 1.697056 -1.697056) (size 0.8 0.8) (drill 0.5) (layers *.Cu *.Mask) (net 6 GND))
  (pad 1 thru_hole circle (at 0 -2.4) (size 0.8 0.8) (drill 0.5) (layers *.Cu *.Mask) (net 6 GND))
  (pad 1 thru_hole circle (at -1.697056 -1.697056) (size 0.8 0.8) (drill 0.5) (layers *.Cu *.Mask) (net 6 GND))
  (pad 1 thru_hole circle (at -2.4 0) (size 0.8 0.8) (drill 0.5) (layers *.Cu *.Mask) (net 6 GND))
  (pad 1 thru_hole circle (at -1.697056 1.697056) (size 0.8 0.8) (drill 0.5) (layers *.Cu *.Mask) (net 6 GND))
  (pad 1 thru_hole circle (at 0 2.4) (size 0.8 0.8) (drill 0.5) (layers *.Cu *.Mask) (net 6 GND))
  (pad 1 thru_hole circle (at 1.697056 1.697056) (size 0.8 0.8) (drill 0.5) (layers *.Cu *.Mask) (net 6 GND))
  (pad 1 thru_hole circle (at 2.4 0) (size 0.8 0.8) (drill 0.5) (layers *.Cu *.Mask) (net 6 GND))
  (pad 1 thru_hole circle (at 0 0) (size 6.4 6.4) (drill 3.2) (layers *.Cu *.Mask) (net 6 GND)))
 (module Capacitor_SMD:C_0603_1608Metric (layer B.Cu) (at 31.5722 19.1516 270)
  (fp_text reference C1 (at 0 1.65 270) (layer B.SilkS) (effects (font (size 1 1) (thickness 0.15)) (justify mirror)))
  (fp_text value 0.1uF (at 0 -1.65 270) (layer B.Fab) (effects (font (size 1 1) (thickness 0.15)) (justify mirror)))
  (pad 2 smd rect (at 0.875 0 270) (size 0.67 1) (layers B.Cu B.Paste B.Mask) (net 6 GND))
  (pad 1 smd rect (at -0.875 0 270) (size 0.67 1) (layers B.Cu B.Paste B.Mask) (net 3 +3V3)))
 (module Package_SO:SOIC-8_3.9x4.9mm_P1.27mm (layer B.Cu) (at 36.5836 20.3962 180)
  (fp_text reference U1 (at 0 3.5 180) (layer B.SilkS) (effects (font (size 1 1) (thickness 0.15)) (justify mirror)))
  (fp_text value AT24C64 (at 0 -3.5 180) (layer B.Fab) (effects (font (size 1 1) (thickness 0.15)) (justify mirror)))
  (pad 1 smd rect (at -2.7 1.905 180) (size 1.55 0.6) (layers B.Cu B.Paste B.Mask) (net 6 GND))
  (pad 2 smd rect (at -2.7 0.635 180) (size 1.55 0.6) (layers B.Cu B.Paste B.Mask) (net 6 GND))
  (pad 3 smd rect (at -2.7 -0.635 180) (size 1.55 0.6) (layers B.Cu B.Paste B.Mask) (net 6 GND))
  (pad 4 smd rect (at -2.7 -1.905 180) (size 1.55 0.6) (layers B.Cu B.Paste B.Mask) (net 6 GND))
  (pad 5 smd rect (at 2.7 -1.905 180) (size 1.55 0.6) (layers B.Cu B.Paste B.Mask) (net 9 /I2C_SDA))
  (pad 6 smd rect (at 2.7 -0.635 180) (size 1.55 0.6) (layers B.Cu B.Paste B.Mask) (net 10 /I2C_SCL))
  (pad 7 smd rect (at 2.7 0.635 180) (size 1.55 0.6) (layers B.Cu B.Paste B.Mask) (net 6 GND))
  (pad 8 smd rect (at 2.7 1.905 180) (size 1.55 0.6) (layers B.Cu B.Paste B.Mask) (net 3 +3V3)))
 (gr_circle (center 22.500537 63.84) (end 21.800537 63.84) (layer Edge.Cuts) (width 0))
 (gr_line (start 27.5 0) (end 40 0) (layer Edge.Cuts) (width 0))
 (gr_arc (start 27.5 1.5) (end 27.5 0) (angle -90) (layer Edge.Cuts) (width 0))
 (gr_arc (start 17.5 1.5) (end 19 1.5) (angle -90) (layer Edge.Cuts) (width 0))
 (gr_line (start 6.5 0) (end 17.5 0) (layer Edge.Cuts) (width 0))
 (gr_arc (start 6.5 1.5) (end 6.5 0) (angle -90) (layer Edge.Cuts) (width 0))
 (gr_arc (start 27.5 73.5) (end 26 73.5) (angle -90) (layer Edge.Cuts) (width 0))
 (gr_arc (start 1.5 68.5) (end 0 68.5) (angle -90) (layer Edge.Cuts) (width 0))
 (gr_arc (start 1.5 6.5) (end 1.5 5) (angle -90) (layer Edge.Cuts) (width 0))
 (gr_line (start 0 68.5) (end 0 6.5) (layer Edge.Cuts) (width 0))
 (gr_arc (start 1.5 73.5) (end 5 73.5) (angle -90) (layer Edge.Cuts) (width 0))
 (gr_arc (start 6.5 73.5) (end 5 73.5) (angle -90) (layer Edge.Cuts) (width 0))
 (gr_line (start 45 5) (end 45 70) (layer Edge.Cuts) (width 0))
 (gr_line (start 17.5 75) (end 6.5 75) (layer Edge.Cuts) (width 0))
 (gr_arc (start 40 70) (end 40 75) (angle -90) (layer Edge.Cuts) (width 0))
 (gr_arc (start 22.5 73.5) (end 26 73.5) (angle -180) (layer Edge.Cuts) (width 0))
 (gr_arc (start 1.5 1.5) (end 1.5 5) (angle -90) (layer Edge.Cuts) (width 0))
 (gr_line (start 40 75) (end 27.5 75) (layer Edge.Cuts) (width 0))
 (gr_arc (start 17.5 73.5) (end 17.5 75) (angle -90) (layer Edge.Cuts) (width 0))
 (gr_arc (start 40 5) (end 45 5) (angle -90) (layer Edge.Cuts) (width 0))
 (gr_arc (start 22.5 1.5) (end 19 1.5) (angle -180) (layer Edge.Cuts) (width 0))
 (segment (start 20.55 12.735) (end 22 12.735) (width 0.25) (layer F.Cu) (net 1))
 (segment (start 22 12.735) (end 24.45 12.735) (width 0.25) (layer F.Cu) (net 1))
 (segment (start 20.7 12.735) (end 24.3 12.735) (width 0.25) (layer B.Cu) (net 1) (status 30))
 (segment (start 24.3 14.005) (end 20.7 14.005) (width 0.25) (layer B.Cu) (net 2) (status 30))
 (segment (start 24.45 14.005) (end 20.55 14.005) (width 0.25) (layer F.Cu) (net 2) (status 30))
 (segment (start 24.3 16.545) (end 20.7 16.545) (width 0.25) (layer B.Cu) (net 4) (status 30))
 (segment (start 20.7 17.815) (end 24.3 17.815) (width 0.25) (layer B.Cu) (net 5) (status 30))
 (segment (start 20.55 17.815) (end 24.45 17.815) (width 0.25) (layer F.Cu) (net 5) (status 30))
 (segment (start 20.7 21.625) (end 22.514 21.625) (width 0.25) (layer B.Cu) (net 9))
 (segment (start 22.514 21.625) (end 23.183999 22.294999) (width 0.25) (layer B.Cu) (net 9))
 (segment (start 23.183999 22.294999) (end 28.374398 22.294999) (width 0.25) (layer B.Cu) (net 9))
 (segment (start 28.374398 22.294999) (end 29.21 23.130601) (width 0.25) (layer B.Cu) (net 9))
 (segment (start 29.21 23.130601) (end 30.099 23.130601) (width 0.25) (layer B.Cu) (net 9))
 (segment (start 30.099 23.130601) (end 31.877 23.130601) (width 0.25) (layer B.Cu) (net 9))
 (segment (start 31.877 23.130601) (end 32.579199 23.130601) (width 0.25) (layer B.Cu) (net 9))
 (segment (start 31.8897 22.5806) (end 31.8897 23.117901) (width 0.25) (layer B.Cu) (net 9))
 (segment (start 31.8897 23.117901) (end 31.877 23.130601) (width 0.25) (layer B.Cu) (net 9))
 (segment (start 32.579199 23.130601) (end 33.4086 22.3012) (width 0.25) (layer B.Cu) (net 9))
 (segment (start 33.4086 22.3012) (end 33.8836 22.3012) (width 0.25) (layer B.Cu) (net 9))
 (segment (start 24.3 21.625) (end 29.118 21.625) (width 0.25) (layer B.Cu) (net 10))
 (segment (start 29.118 21.625) (end 29.464 21.971) (width 0.25) (layer B.Cu) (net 10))
 (segment (start 29.464 21.971) (end 29.972 21.971) (width 0.25) (layer B.Cu) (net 10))
 (segment (start 29.972 21.971) (end 31.877 21.971) (width 0.25) (layer B.Cu) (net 10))
 (segment (start 31.877 21.971) (end 32.4688 21.971) (width 0.25) (layer B.Cu) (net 10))
 (segment (start 31.8897 21.3614) (end 31.8897 21.9583) (width 0.25) (layer B.Cu) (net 10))
 (segment (start 31.8897 21.9583) (end 31.877 21.971) (width 0.25) (layer B.Cu) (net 10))
 (segment (start 32.4688 21.971) (end 33.4086 21.0312) (width 0.25) (layer B.Cu) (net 10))
 (segment (start 33.4086 21.0312) (end 33.8836 21.0312) (width 0.25) (layer B.Cu) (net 10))
 (segment (start 24.3 19.085) (end 28.6494 19.085) (width 0.25) (layer B.Cu) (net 6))
 (segment (start 28.6494 19.085) (end 29.591 20.0266) (width 0.25) (layer B.Cu) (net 6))
 (segment (start 29.591 20.0266) (end 31.5722 20.0266) (width 0.25) (layer B.Cu) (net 6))
 (segment (start 32.4244 20.0266) (end 32.6898 19.7612) (width 0.25) (layer B.Cu) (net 6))
 (segment (start 32.6898 19.7612) (end 33.8836 19.7612) (width 0.25) (layer B.Cu) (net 6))
 (segment (start 31.5722 20.0266) (end 32.4244 20.0266) (width 0.25) (layer B.Cu) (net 6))
 (segment (start 33.8836 19.7612) (end 34.9086 19.7612) (width 0.25) (layer B.Cu) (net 6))
 (segment (start 34.9086 19.7612) (end 39.2836 19.7612) (width 0.25) (layer B.Cu) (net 6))
 (segment (start 39.2836 18.4912) (end 39.2836 22.3012) (width 0.25) (layer B.Cu) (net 6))
 (segment (start 24.3 19.085) (end 23 19.085) (width 0.25) (layer B.Cu) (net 6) (status 10))
 (segment (start 23 19.085) (end 20.7 19.085) (width 0.25) (layer B.Cu) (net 6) (status 20))
 (segment (start 26.832 15.275) (end 29.8336 18.2766) (width 0.25) (layer B.Cu) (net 3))
 (segment (start 29.8336 18.2766) (end 31.5722 18.2766) (width 0.25) (layer B.Cu) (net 3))
 (segment (start 24.3 15.275) (end 26.832 15.275) (width 0.25) (layer B.Cu) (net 3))
 (segment (start 32.3736 18.2766) (end 32.5882 18.4912) (width 0.25) (layer B.Cu) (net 3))
 (segment (start 32.5882 18.4912) (end 33.8836 18.4912) (width 0.25) (layer B.Cu) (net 3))
 (segment (start 31.5722 18.2766) (end 32.3736 18.2766) (width 0.25) (layer B.Cu) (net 3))
 (segment (start 20.7 15.275) (end 24.3 15.275) (width 0.25) (layer B.Cu) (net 3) (status 30))
 (segment (start 20.55 15.275) (end 24.45 15.275) (width 0.25) (layer F.Cu) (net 3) (status 30))
 (segment (start 24.45 16.545) (end 23 16.545) (width 0.25) (layer F.Cu) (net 4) (status 10))
 (segment (start 23 16.545) (end 20.55 16.545) (width 0.25) (layer F.Cu) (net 4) (status 20))
 (segment (start 20.55 19.085) (end 24.45 19.085) (width 0.25) (layer F.Cu) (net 6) (status 30)))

